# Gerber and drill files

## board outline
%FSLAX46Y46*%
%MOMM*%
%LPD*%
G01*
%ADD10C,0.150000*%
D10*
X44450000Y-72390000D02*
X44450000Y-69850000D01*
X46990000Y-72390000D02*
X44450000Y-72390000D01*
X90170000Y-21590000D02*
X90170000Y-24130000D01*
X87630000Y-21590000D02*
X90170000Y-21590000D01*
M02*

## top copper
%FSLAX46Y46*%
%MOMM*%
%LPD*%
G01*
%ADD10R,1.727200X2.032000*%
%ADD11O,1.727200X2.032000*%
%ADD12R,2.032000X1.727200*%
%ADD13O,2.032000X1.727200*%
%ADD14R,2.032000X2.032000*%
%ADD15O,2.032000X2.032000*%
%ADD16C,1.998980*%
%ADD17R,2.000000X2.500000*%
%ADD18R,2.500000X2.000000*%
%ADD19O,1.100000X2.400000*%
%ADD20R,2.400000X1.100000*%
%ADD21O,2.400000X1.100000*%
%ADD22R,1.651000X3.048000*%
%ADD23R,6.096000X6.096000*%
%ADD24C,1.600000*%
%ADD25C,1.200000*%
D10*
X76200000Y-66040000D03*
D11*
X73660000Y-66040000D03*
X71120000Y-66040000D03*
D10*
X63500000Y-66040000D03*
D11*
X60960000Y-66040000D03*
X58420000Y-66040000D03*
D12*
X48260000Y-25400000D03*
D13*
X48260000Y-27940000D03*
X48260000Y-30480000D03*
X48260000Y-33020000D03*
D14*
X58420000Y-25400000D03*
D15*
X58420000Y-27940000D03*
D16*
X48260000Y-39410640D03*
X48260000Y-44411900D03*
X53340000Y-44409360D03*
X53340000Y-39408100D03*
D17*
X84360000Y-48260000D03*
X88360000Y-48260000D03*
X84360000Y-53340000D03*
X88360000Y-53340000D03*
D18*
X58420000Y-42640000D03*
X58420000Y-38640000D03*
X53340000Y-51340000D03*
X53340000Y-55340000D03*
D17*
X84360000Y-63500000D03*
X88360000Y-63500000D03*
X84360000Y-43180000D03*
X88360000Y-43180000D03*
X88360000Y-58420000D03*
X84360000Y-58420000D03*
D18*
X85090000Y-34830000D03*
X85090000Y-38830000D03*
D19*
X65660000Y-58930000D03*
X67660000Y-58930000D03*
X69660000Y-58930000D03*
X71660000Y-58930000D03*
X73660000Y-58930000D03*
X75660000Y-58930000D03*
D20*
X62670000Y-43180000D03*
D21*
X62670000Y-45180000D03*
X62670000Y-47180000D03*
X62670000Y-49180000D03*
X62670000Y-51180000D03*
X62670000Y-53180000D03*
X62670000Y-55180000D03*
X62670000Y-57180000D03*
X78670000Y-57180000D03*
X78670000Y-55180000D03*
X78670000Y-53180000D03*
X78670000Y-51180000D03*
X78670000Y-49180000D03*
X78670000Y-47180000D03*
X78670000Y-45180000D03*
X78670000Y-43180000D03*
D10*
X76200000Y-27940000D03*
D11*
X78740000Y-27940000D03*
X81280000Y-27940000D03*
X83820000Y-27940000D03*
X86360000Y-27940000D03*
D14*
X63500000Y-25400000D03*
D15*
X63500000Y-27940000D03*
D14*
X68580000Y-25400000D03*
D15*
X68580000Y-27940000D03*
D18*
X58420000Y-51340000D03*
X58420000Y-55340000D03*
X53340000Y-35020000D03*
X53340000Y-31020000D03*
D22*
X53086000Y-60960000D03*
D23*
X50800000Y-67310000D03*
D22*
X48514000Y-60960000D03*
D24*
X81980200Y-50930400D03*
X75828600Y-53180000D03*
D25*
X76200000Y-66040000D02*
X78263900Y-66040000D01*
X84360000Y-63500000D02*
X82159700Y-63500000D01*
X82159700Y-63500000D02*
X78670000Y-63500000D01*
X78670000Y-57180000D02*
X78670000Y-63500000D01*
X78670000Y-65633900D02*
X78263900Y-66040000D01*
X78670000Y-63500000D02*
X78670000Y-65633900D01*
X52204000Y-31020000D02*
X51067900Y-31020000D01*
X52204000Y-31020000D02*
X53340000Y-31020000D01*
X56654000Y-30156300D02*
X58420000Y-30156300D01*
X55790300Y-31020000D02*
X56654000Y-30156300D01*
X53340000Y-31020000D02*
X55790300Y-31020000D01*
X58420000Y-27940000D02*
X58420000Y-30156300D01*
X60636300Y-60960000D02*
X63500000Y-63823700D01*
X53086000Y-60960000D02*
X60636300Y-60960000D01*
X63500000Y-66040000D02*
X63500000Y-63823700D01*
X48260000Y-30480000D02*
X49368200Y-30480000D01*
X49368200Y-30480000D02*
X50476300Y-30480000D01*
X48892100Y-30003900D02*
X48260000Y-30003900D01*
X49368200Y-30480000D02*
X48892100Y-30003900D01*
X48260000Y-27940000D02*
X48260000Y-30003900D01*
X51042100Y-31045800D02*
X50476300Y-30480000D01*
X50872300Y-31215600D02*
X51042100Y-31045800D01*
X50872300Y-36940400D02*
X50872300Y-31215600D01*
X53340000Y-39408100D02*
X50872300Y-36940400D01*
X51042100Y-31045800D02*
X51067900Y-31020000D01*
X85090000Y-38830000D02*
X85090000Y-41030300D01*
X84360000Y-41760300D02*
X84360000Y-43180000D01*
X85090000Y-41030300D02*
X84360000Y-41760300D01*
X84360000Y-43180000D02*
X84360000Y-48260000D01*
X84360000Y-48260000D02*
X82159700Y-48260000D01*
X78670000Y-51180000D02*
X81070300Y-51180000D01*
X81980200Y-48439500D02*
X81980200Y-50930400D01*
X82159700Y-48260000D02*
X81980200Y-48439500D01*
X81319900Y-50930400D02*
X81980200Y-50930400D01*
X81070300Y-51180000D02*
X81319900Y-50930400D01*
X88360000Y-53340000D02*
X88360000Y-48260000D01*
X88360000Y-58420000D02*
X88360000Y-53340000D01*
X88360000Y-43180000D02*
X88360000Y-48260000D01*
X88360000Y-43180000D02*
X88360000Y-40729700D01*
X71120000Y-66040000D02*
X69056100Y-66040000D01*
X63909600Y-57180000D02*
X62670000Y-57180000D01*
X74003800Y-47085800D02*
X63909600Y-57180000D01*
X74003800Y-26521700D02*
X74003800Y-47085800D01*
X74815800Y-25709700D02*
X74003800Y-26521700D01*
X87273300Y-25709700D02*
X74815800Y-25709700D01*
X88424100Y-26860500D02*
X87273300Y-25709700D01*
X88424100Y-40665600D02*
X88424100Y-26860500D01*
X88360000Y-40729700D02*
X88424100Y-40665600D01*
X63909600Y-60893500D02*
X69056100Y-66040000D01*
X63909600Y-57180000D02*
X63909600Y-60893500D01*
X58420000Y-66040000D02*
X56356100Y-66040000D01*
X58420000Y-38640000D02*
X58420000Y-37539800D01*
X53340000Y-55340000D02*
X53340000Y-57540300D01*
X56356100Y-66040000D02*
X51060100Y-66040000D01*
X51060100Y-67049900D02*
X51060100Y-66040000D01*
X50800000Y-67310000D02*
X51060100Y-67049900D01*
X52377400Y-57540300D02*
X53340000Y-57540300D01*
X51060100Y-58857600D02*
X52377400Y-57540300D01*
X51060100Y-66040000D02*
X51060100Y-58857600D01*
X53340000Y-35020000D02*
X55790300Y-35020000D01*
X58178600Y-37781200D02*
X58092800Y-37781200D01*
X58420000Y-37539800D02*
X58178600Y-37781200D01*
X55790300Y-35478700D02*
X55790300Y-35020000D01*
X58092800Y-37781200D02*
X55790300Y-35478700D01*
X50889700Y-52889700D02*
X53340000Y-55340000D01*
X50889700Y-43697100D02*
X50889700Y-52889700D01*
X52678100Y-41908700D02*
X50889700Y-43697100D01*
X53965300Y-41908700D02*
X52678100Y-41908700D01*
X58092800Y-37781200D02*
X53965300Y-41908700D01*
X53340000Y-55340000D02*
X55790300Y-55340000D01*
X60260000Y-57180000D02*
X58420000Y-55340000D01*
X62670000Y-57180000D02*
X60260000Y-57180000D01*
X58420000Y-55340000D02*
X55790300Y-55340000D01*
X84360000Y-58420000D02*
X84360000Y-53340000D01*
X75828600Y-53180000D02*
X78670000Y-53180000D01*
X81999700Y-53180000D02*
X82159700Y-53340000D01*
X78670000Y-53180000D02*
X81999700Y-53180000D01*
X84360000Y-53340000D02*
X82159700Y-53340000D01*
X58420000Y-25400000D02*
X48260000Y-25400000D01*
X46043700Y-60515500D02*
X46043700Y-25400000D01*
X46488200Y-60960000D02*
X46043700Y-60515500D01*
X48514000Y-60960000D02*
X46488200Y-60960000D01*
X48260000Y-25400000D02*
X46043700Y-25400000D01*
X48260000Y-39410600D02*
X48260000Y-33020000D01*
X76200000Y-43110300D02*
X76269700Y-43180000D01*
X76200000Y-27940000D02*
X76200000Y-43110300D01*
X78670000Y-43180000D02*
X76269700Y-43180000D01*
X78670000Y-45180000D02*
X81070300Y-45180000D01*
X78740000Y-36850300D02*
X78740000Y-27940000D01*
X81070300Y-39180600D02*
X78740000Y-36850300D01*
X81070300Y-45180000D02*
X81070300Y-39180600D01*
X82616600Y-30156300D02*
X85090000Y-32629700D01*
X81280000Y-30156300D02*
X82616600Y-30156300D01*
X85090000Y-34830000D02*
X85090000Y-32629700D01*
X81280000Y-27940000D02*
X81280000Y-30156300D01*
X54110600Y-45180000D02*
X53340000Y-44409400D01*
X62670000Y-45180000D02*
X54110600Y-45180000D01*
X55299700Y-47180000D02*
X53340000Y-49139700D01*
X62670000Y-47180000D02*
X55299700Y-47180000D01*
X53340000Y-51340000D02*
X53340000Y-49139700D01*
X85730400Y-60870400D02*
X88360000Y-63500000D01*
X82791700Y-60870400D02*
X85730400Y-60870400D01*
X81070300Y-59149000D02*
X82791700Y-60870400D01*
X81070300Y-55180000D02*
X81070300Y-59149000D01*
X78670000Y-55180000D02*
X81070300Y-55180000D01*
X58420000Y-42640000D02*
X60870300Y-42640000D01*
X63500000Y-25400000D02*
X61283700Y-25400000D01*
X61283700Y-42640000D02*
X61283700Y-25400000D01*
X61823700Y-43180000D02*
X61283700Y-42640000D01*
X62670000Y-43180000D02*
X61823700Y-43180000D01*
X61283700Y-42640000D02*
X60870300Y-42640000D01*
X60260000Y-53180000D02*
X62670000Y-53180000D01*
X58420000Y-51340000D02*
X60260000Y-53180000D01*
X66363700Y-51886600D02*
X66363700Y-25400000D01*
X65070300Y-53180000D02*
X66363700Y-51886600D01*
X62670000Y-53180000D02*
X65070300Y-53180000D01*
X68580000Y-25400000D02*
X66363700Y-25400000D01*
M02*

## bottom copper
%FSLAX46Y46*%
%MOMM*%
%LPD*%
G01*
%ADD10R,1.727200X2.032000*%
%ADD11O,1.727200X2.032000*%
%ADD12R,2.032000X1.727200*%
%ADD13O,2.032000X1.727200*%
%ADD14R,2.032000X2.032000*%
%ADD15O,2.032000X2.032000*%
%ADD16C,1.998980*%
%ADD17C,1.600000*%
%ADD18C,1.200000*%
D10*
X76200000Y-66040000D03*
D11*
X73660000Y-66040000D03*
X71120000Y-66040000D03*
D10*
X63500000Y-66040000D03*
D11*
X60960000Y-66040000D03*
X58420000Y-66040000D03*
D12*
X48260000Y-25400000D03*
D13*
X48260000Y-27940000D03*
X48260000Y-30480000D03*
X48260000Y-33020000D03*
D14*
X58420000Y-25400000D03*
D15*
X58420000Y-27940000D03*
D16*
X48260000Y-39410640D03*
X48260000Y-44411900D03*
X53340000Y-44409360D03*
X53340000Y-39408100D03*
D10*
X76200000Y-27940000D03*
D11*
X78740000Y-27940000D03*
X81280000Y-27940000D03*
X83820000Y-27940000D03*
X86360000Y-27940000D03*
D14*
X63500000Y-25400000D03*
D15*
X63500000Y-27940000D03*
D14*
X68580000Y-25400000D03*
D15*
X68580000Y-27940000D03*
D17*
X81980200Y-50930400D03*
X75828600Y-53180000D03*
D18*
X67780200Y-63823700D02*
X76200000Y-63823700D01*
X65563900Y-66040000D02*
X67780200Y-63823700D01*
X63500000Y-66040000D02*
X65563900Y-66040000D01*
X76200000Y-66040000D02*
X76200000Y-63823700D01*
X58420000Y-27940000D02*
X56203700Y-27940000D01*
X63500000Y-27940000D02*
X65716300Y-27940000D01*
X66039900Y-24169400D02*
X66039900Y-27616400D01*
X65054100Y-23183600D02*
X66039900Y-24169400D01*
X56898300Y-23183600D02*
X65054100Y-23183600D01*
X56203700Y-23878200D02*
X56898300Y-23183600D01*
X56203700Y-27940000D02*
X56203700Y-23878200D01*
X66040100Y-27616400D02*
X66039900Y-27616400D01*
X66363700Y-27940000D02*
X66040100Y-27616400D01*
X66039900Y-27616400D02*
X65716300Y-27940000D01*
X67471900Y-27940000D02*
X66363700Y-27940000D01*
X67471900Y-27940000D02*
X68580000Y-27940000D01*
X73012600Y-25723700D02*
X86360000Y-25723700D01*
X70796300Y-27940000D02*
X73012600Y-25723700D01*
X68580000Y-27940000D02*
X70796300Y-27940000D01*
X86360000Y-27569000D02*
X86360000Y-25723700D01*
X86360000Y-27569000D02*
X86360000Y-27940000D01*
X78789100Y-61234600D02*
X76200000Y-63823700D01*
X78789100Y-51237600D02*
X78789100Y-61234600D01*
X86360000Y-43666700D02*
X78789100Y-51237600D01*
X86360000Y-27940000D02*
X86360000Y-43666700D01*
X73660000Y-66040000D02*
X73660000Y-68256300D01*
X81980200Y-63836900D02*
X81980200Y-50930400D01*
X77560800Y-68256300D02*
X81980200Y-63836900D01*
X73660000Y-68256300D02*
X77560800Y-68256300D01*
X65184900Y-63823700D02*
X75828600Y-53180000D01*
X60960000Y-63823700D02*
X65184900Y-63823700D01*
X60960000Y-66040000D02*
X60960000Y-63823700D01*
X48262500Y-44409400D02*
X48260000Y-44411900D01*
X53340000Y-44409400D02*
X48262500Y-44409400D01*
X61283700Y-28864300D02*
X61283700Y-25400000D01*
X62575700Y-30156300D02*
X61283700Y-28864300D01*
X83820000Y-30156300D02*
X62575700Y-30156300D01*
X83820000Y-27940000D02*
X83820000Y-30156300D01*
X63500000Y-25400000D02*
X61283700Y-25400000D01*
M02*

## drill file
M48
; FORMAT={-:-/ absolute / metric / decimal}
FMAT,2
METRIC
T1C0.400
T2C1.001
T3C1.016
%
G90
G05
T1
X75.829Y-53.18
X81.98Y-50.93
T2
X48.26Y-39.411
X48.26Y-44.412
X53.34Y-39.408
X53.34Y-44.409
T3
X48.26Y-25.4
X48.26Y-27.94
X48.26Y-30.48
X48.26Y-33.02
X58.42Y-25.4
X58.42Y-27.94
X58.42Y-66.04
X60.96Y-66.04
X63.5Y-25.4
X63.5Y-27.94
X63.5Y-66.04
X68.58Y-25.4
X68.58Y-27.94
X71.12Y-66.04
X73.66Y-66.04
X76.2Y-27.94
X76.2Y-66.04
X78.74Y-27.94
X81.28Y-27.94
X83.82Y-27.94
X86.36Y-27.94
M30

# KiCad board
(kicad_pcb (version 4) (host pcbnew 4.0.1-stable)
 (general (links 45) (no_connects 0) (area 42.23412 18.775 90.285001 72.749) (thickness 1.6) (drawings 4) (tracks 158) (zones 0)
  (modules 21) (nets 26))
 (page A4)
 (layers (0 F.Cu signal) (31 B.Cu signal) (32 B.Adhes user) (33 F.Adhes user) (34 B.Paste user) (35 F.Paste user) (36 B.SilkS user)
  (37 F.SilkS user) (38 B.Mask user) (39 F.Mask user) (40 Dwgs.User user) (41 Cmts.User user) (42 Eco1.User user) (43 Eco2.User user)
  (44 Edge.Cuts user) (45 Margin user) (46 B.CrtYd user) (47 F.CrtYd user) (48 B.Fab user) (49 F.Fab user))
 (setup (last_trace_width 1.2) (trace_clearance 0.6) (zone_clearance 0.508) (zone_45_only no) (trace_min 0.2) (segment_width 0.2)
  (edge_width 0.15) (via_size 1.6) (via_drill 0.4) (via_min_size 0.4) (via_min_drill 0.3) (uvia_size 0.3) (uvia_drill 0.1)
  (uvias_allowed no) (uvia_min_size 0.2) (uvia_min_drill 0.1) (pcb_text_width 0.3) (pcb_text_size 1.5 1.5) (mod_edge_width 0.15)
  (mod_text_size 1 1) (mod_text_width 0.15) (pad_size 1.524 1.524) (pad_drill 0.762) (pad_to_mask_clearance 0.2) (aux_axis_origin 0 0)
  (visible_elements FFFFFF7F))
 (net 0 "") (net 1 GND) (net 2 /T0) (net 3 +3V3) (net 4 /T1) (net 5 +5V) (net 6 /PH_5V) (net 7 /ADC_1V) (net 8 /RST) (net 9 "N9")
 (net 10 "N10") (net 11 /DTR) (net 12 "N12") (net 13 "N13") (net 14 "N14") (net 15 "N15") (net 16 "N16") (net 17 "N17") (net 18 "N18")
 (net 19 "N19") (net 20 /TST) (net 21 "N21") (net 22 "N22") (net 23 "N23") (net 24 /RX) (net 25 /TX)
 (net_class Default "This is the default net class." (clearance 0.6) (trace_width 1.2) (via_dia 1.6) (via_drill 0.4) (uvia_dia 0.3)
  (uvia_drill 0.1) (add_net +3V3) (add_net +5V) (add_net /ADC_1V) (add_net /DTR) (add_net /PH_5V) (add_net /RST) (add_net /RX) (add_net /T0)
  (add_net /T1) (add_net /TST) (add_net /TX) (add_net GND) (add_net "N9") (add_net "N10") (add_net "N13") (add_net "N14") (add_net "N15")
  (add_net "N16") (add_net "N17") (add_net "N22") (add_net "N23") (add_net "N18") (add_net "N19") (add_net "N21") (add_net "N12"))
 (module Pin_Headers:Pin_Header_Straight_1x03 (layer F.Cu) (at 76.2 66.04 270)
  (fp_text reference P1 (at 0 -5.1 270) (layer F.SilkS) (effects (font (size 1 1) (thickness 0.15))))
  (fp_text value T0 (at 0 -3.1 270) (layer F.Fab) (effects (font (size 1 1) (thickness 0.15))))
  (pad 1 thru_hole rect (at 0 0 270) (size 2.032 1.7272) (drill 1.016) (layers *.Cu *.Mask F.SilkS) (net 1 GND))
  (pad 2 thru_hole oval (at 0 2.54 270) (size 2.032 1.7272) (drill 1.016) (layers *.Cu *.Mask F.SilkS) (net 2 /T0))
  (pad 3 thru_hole oval (at 0 5.08 270) (size 2.032 1.7272) (drill 1.016) (layers *.Cu *.Mask F.SilkS) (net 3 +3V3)))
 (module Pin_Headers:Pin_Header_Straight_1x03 (layer F.Cu) (at 63.5 66.04 270)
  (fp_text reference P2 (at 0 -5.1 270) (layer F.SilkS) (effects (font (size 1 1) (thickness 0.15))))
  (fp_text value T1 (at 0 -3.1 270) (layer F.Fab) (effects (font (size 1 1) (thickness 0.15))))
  (pad 1 thru_hole rect (at 0 0 270) (size 2.032 1.7272) (drill 1.016) (layers *.Cu *.Mask F.SilkS) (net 1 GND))
  (pad 2 thru_hole oval (at 0 2.54 270) (size 2.032 1.7272) (drill 1.016) (layers *.Cu *.Mask F.SilkS) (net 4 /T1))
  (pad 3 thru_hole oval (at 0 5.08 270) (size 2.032 1.7272) (drill 1.016) (layers *.Cu *.Mask F.SilkS) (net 3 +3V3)))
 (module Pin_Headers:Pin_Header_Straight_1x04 (layer F.Cu) (at 48.26 25.4)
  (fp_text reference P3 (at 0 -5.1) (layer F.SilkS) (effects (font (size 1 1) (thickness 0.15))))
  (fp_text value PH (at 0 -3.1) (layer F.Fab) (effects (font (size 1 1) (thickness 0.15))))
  (pad 1 thru_hole rect (at 0 0) (size 2.032 1.7272) (drill 1.016) (layers *.Cu *.Mask F.SilkS) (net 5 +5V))
  (pad 2 thru_hole oval (at 0 2.54) (size 2.032 1.7272) (drill 1.016) (layers *.Cu *.Mask F.SilkS) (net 1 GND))
  (pad 3 thru_hole oval (at 0 5.08) (size 2.032 1.7272) (drill 1.016) (layers *.Cu *.Mask F.SilkS) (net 1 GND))
  (pad 4 thru_hole oval (at 0 7.62) (size 2.032 1.7272) (drill 1.016) (layers *.Cu *.Mask F.SilkS) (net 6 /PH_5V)))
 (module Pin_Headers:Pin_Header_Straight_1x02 (layer F.Cu) (at 58.42 25.4)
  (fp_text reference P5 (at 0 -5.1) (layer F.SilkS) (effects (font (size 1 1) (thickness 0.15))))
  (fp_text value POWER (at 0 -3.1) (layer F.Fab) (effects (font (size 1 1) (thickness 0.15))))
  (pad 1 thru_hole rect (at 0 0) (size 2.032 2.032) (drill 1.016) (layers *.Cu *.Mask F.SilkS) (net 5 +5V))
  (pad 2 thru_hole oval (at 0 2.54) (size 2.032 2.032) (drill 1.016) (layers *.Cu *.Mask F.SilkS) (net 1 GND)))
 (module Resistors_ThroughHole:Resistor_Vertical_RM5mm (layer F.Cu) (at 48.26 41.91 270)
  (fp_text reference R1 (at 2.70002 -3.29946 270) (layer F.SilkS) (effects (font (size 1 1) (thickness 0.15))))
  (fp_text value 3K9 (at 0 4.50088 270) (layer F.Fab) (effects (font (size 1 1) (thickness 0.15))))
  (pad 1 thru_hole circle (at -2.49936 0 270) (size 1.99898 1.99898) (drill 1.00076) (layers *.Cu *.SilkS *.Mask) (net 6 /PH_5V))
  (pad 2 thru_hole circle (at 2.5019 0 270) (size 1.99898 1.99898) (drill 1.00076) (layers *.Cu *.SilkS *.Mask) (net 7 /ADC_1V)))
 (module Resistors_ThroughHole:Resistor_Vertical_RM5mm (layer F.Cu) (at 53.34 41.91 90)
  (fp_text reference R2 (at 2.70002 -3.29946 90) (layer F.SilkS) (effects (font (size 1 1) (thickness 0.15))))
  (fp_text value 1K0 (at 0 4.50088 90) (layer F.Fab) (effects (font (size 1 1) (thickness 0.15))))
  (pad 1 thru_hole circle (at -2.49936 0 90) (size 1.99898 1.99898) (drill 1.00076) (layers *.Cu *.SilkS *.Mask) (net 7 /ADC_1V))
  (pad 2 thru_hole circle (at 2.5019 0 90) (size 1.99898 1.99898) (drill 1.00076) (layers *.Cu *.SilkS *.Mask) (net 1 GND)))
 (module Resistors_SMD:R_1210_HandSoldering (layer F.Cu) (at 86.36 48.26)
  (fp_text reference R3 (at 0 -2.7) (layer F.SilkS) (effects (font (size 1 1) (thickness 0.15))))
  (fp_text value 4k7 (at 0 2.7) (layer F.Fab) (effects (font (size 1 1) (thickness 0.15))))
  (pad 1 smd rect (at -2 0) (size 2 2.5) (layers F.Cu F.Paste F.Mask) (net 2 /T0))
  (pad 2 smd rect (at 2 0) (size 2 2.5) (layers F.Cu F.Paste F.Mask) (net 3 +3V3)))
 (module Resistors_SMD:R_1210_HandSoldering (layer F.Cu) (at 86.36 53.34)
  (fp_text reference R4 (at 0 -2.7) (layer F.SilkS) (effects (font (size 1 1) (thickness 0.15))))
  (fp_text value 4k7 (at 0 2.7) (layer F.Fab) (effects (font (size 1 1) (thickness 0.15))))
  (pad 1 smd rect (at -2 0) (size 2 2.5) (layers F.Cu F.Paste F.Mask) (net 4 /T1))
  (pad 2 smd rect (at 2 0) (size 2 2.5) (layers F.Cu F.Paste F.Mask) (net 3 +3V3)))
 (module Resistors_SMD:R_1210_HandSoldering (layer F.Cu) (at 58.42 40.64 90)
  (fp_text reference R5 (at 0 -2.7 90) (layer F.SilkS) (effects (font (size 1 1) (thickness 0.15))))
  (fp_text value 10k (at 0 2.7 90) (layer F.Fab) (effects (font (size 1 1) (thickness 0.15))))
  (pad 1 smd rect (at -2 0 90) (size 2 2.5) (layers F.Cu F.Paste F.Mask) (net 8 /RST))
  (pad 2 smd rect (at 2 0 90) (size 2 2.5) (layers F.Cu F.Paste F.Mask) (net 3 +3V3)))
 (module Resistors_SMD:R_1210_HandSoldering (layer F.Cu) (at 53.34 53.34 270)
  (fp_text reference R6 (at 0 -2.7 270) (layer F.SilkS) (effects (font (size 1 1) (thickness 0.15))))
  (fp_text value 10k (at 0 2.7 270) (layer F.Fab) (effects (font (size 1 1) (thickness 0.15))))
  (pad 1 smd rect (at -2 0 270) (size 2 2.5) (layers F.Cu F.Paste F.Mask) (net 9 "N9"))
  (pad 2 smd rect (at 2 0 270) (size 2 2.5) (layers F.Cu F.Paste F.Mask) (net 3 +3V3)))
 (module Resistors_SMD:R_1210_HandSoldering (layer F.Cu) (at 86.36 63.5)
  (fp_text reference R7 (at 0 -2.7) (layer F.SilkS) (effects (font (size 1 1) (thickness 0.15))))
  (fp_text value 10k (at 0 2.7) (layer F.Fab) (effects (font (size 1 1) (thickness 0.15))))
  (pad 1 smd rect (at -2 0) (size 2 2.5) (layers F.Cu F.Paste F.Mask) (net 1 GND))
  (pad 2 smd rect (at 2 0) (size 2 2.5) (layers F.Cu F.Paste F.Mask) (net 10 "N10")))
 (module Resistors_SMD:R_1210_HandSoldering (layer F.Cu) (at 86.36 43.18)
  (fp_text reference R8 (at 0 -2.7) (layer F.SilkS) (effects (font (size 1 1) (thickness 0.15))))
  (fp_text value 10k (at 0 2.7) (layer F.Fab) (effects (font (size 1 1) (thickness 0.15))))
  (pad 1 smd rect (at -2 0) (size 2 2.5) (layers F.Cu F.Paste F.Mask) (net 2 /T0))
  (pad 2 smd rect (at 2 0) (size 2 2.5) (layers F.Cu F.Paste F.Mask) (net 3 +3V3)))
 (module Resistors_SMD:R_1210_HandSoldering (layer F.Cu) (at 86.36 58.42 180)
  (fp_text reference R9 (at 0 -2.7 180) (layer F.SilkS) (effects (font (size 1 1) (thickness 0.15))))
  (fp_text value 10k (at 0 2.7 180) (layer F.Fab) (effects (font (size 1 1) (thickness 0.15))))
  (pad 1 smd rect (at -2 0 180) (size 2 2.5) (layers F.Cu F.Paste F.Mask) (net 3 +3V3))
  (pad 2 smd rect (at 2 0 180) (size 2 2.5) (layers F.Cu F.Paste F.Mask) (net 4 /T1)))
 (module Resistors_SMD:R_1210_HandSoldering (layer F.Cu) (at 85.09 36.83 270)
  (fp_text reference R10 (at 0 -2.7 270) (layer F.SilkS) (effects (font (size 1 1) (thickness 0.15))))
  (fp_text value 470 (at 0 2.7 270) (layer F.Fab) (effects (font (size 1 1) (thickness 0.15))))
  (pad 1 smd rect (at -2 0 270) (size 2 2.5) (layers F.Cu F.Paste F.Mask) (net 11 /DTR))
  (pad 2 smd rect (at 2 0 270) (size 2 2.5) (layers F.Cu F.Paste F.Mask) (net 2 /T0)))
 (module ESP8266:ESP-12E (layer F.Cu) (at 62.67 43.18)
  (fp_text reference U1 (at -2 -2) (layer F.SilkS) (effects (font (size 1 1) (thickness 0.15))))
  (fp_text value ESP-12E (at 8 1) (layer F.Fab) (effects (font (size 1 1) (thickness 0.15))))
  (pad 9 smd oval (at 2.99 15.75 90) (size 2.4 1.1) (layers F.Cu F.Paste F.Mask) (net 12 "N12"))
  (pad 10 smd oval (at 4.99 15.75 90) (size 2.4 1.1) (layers F.Cu F.Paste F.Mask) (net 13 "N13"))
  (pad 11 smd oval (at 6.99 15.75 90) (size 2.4 1.1) (layers F.Cu F.Paste F.Mask) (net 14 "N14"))
  (pad 12 smd oval (at 8.99 15.75 90) (size 2.4 1.1) (layers F.Cu F.Paste F.Mask) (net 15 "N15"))
  (pad 13 smd oval (at 10.99 15.75 90) (size 2.4 1.1) (layers F.Cu F.Paste F.Mask) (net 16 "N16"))
  (pad 14 smd oval (at 12.99 15.75 90) (size 2.4 1.1) (layers F.Cu F.Paste F.Mask) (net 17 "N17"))
  (pad 1 smd rect (at 0 0) (size 2.4 1.1) (layers F.Cu F.Paste F.Mask) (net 8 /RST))
  (pad 2 smd oval (at 0 2) (size 2.4 1.1) (layers F.Cu F.Paste F.Mask) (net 7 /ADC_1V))
  (pad 3 smd oval (at 0 4) (size 2.4 1.1) (layers F.Cu F.Paste F.Mask) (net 9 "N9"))
  (pad 4 smd oval (at 0 6) (size 2.4 1.1) (layers F.Cu F.Paste F.Mask) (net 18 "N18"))
  (pad 5 smd oval (at 0 8) (size 2.4 1.1) (layers F.Cu F.Paste F.Mask) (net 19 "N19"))
  (pad 6 smd oval (at 0 10) (size 2.4 1.1) (layers F.Cu F.Paste F.Mask) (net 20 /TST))
  (pad 7 smd oval (at 0 12) (size 2.4 1.1) (layers F.Cu F.Paste F.Mask) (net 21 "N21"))
  (pad 8 smd oval (at 0 14) (size 2.4 1.1) (layers F.Cu F.Paste F.Mask) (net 3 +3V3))
  (pad 15 smd oval (at 16 14) (size 2.4 1.1) (layers F.Cu F.Paste F.Mask) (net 1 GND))
  (pad 16 smd oval (at 16 12) (size 2.4 1.1) (layers F.Cu F.Paste F.Mask) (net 10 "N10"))
  (pad 17 smd oval (at 16 10) (size 2.4 1.1) (layers F.Cu F.Paste F.Mask) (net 4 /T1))
  (pad 18 smd oval (at 16 8) (size 2.4 1.1) (layers F.Cu F.Paste F.Mask) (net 2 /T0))
  (pad 19 smd oval (at 16 6) (size 2.4 1.1) (layers F.Cu F.Paste F.Mask) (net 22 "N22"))
  (pad 20 smd oval (at 16 4) (size 2.4 1.1) (layers F.Cu F.Paste F.Mask) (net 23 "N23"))
  (pad 21 smd oval (at 16 2) (size 2.4 1.1) (layers F.Cu F.Paste F.Mask) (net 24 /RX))
  (pad 22 smd oval (at 16 0) (size 2.4 1.1) (layers F.Cu F.Paste F.Mask) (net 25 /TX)))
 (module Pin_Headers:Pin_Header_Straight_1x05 (layer F.Cu) (at 76.2 27.94 90)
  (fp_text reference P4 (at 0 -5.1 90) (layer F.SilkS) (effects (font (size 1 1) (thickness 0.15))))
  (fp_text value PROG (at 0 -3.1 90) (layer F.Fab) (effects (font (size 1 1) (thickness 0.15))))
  (pad 1 thru_hole rect (at 0 0 90) (size 2.032 1.7272) (drill 1.016) (layers *.Cu *.Mask F.SilkS) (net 25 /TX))
  (pad 2 thru_hole oval (at 0 2.54 90) (size 2.032 1.7272) (drill 1.016) (layers *.Cu *.Mask F.SilkS) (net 24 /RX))
  (pad 3 thru_hole oval (at 0 5.08 90) (size 2.032 1.7272) (drill 1.016) (layers *.Cu *.Mask F.SilkS) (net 11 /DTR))
  (pad 4 thru_hole oval (at 0 7.62 90) (size 2.032 1.7272) (drill 1.016) (layers *.Cu *.Mask F.SilkS) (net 8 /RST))
  (pad 5 thru_hole oval (at 0 10.16 90) (size 2.032 1.7272) (drill 1.016) (layers *.Cu *.Mask F.SilkS) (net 1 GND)))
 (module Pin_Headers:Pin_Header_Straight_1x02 (layer F.Cu) (at 63.5 25.4)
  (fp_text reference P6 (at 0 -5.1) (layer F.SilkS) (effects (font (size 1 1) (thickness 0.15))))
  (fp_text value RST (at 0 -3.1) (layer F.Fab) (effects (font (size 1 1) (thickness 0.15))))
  (pad 1 thru_hole rect (at 0 0) (size 2.032 2.032) (drill 1.016) (layers *.Cu *.Mask F.SilkS) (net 8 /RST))
  (pad 2 thru_hole oval (at 0 2.54) (size 2.032 2.032) (drill 1.016) (layers *.Cu *.Mask F.SilkS) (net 1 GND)))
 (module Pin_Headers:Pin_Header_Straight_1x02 (layer F.Cu) (at 68.58 25.4)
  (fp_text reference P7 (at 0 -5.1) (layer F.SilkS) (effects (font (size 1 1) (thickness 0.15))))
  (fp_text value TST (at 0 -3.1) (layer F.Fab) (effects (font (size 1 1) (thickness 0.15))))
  (pad 1 thru_hole rect (at 0 0) (size 2.032 2.032) (drill 1.016) (layers *.Cu *.Mask F.SilkS) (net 20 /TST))
  (pad 2 thru_hole oval (at 0 2.54) (size 2.032 2.032) (drill 1.016) (layers *.Cu *.Mask F.SilkS) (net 1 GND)))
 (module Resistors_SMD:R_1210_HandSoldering (layer F.Cu) (at 58.42 53.34 270)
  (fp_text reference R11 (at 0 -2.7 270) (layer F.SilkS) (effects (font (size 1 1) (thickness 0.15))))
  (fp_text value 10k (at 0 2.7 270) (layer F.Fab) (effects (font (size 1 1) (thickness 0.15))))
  (pad 1 smd rect (at -2 0 270) (size 2 2.5) (layers F.Cu F.Paste F.Mask) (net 20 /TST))
  (pad 2 smd rect (at 2 0 270) (size 2 2.5) (layers F.Cu F.Paste F.Mask) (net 3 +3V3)))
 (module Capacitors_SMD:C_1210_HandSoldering (layer F.Cu) (at 53.34 33.02 90)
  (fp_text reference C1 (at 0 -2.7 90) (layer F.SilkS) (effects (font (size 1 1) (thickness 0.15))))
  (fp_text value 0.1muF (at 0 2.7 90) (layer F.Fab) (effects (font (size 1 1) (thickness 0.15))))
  (pad 1 smd rect (at -2 0 90) (size 2 2.5) (layers F.Cu F.Paste F.Mask) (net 3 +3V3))
  (pad 2 smd rect (at 2 0 90) (size 2 2.5) (layers F.Cu F.Paste F.Mask) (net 1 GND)))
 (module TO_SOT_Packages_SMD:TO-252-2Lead (layer F.Cu) (at 50.8 60.96 180)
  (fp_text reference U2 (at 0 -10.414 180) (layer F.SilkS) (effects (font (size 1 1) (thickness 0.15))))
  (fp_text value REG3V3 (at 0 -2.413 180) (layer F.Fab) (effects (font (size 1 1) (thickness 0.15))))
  (pad 1 smd rect (at -2.286 0 180) (size 1.651 3.048) (layers F.Cu F.Paste F.Mask) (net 1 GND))
  (pad 2 smd rect (at 0 -6.35 180) (size 6.096 6.096) (layers F.Cu F.Paste F.Mask) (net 3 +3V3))
  (pad 3 smd rect (at 2.286 0 180) (size 1.651 3.048) (layers F.Cu F.Paste F.Mask) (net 5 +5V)))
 (gr_line (start 44.45 72.39) (end 44.45 69.85) (angle 90) (layer Edge.Cuts) (width 0.15))
 (gr_line (start 46.99 72.39) (end 44.45 72.39) (angle 90) (layer Edge.Cuts) (width 0.15))
 (gr_line (start 90.17 21.59) (end 90.17 24.13) (angle 90) (layer Edge.Cuts) (width 0.15))
 (gr_line (start 87.63 21.59) (end 90.17 21.59) (angle 90) (layer Edge.Cuts) (width 0.15))
 (segment (start 76.2 66.04) (end 78.2639 66.04) (width 1.2) (layer F.Cu) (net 1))
 (segment (start 84.36 63.5) (end 82.1597 63.5) (width 1.2) (layer F.Cu) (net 1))
 (segment (start 82.1597 63.5) (end 78.67 63.5) (width 1.2) (layer F.Cu) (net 1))
 (segment (start 78.67 57.18) (end 78.67 63.5) (width 1.2) (layer F.Cu) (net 1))
 (segment (start 78.67 65.6339) (end 78.2639 66.04) (width 1.2) (layer F.Cu) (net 1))
 (segment (start 78.67 63.5) (end 78.67 65.6339) (width 1.2) (layer F.Cu) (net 1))
 (segment (start 67.7802 63.8237) (end 76.2 63.8237) (width 1.2) (layer B.Cu) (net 1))
 (segment (start 65.5639 66.04) (end 67.7802 63.8237) (width 1.2) (layer B.Cu) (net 1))
 (segment (start 63.5 66.04) (end 65.5639 66.04) (width 1.2) (layer B.Cu) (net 1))
 (segment (start 76.2 66.04) (end 76.2 63.8237) (width 1.2) (layer B.Cu) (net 1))
 (segment (start 58.42 27.94) (end 56.2037 27.94) (width 1.2) (layer B.Cu) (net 1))
 (segment (start 63.5 27.94) (end 65.7163 27.94) (width 1.2) (layer B.Cu) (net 1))
 (segment (start 66.0399 24.1694) (end 66.0399 27.6164) (width 1.2) (layer B.Cu) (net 1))
 (segment (start 65.0541 23.1836) (end 66.0399 24.1694) (width 1.2) (layer B.Cu) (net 1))
 (segment (start 56.8983 23.1836) (end 65.0541 23.1836) (width 1.2) (layer B.Cu) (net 1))
 (segment (start 56.2037 23.8782) (end 56.8983 23.1836) (width 1.2) (layer B.Cu) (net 1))
 (segment (start 56.2037 27.94) (end 56.2037 23.8782) (width 1.2) (layer B.Cu) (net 1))
 (segment (start 66.0401 27.6164) (end 66.0399 27.6164) (width 1.2) (layer B.Cu) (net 1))
 (segment (start 66.3637 27.94) (end 66.0401 27.6164) (width 1.2) (layer B.Cu) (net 1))
 (segment (start 66.0399 27.6164) (end 65.7163 27.94) (width 1.2) (layer B.Cu) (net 1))
 (segment (start 67.4719 27.94) (end 66.3637 27.94) (width 1.2) (layer B.Cu) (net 1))
 (segment (start 67.4719 27.94) (end 68.58 27.94) (width 1.2) (layer B.Cu) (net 1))
 (segment (start 73.0126 25.7237) (end 86.36 25.7237) (width 1.2) (layer B.Cu) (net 1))
 (segment (start 70.7963 27.94) (end 73.0126 25.7237) (width 1.2) (layer B.Cu) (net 1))
 (segment (start 68.58 27.94) (end 70.7963 27.94) (width 1.2) (layer B.Cu) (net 1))
 (segment (start 52.204 31.02) (end 51.0679 31.02) (width 1.2) (layer F.Cu) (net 1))
 (segment (start 52.204 31.02) (end 53.34 31.02) (width 1.2) (layer F.Cu) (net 1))
 (segment (start 56.654 30.1563) (end 58.42 30.1563) (width 1.2) (layer F.Cu) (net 1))
 (segment (start 55.7903 31.02) (end 56.654 30.1563) (width 1.2) (layer F.Cu) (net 1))
 (segment (start 53.34 31.02) (end 55.7903 31.02) (width 1.2) (layer F.Cu) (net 1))
 (segment (start 58.42 27.94) (end 58.42 30.1563) (width 1.2) (layer F.Cu) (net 1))
 (segment (start 60.6363 60.96) (end 63.5 63.8237) (width 1.2) (layer F.Cu) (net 1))
 (segment (start 53.086 60.96) (end 60.6363 60.96) (width 1.2) (layer F.Cu) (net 1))
 (segment (start 63.5 66.04) (end 63.5 63.8237) (width 1.2) (layer F.Cu) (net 1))
 (segment (start 86.36 27.569) (end 86.36 25.7237) (width 1.2) (layer B.Cu) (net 1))
 (segment (start 86.36 27.569) (end 86.36 27.94) (width 1.2) (layer B.Cu) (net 1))
 (segment (start 78.7891 61.2346) (end 76.2 63.8237) (width 1.2) (layer B.Cu) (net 1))
 (segment (start 78.7891 51.2376) (end 78.7891 61.2346) (width 1.2) (layer B.Cu) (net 1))
 (segment (start 86.36 43.6667) (end 78.7891 51.2376) (width 1.2) (layer B.Cu) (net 1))
 (segment (start 86.36 27.94) (end 86.36 43.6667) (width 1.2) (layer B.Cu) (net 1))
 (segment (start 48.26 30.48) (end 49.3682 30.48) (width 1.2) (layer F.Cu) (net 1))
 (segment (start 49.3682 30.48) (end 50.4763 30.48) (width 1.2) (layer F.Cu) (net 1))
 (segment (start 48.8921 30.0039) (end 48.26 30.0039) (width 1.2) (layer F.Cu) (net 1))
 (segment (start 49.3682 30.48) (end 48.8921 30.0039) (width 1.2) (layer F.Cu) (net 1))
 (segment (start 48.26 27.94) (end 48.26 30.0039) (width 1.2) (layer F.Cu) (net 1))
 (segment (start 51.0421 31.0458) (end 50.4763 30.48) (width 1.2) (layer F.Cu) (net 1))
 (segment (start 50.8723 31.2156) (end 51.0421 31.0458) (width 1.2) (layer F.Cu) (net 1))
 (segment (start 50.8723 36.9404) (end 50.8723 31.2156) (width 1.2) (layer F.Cu) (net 1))
 (segment (start 53.34 39.4081) (end 50.8723 36.9404) (width 1.2) (layer F.Cu) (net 1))
 (segment (start 51.0421 31.0458) (end 51.0679 31.02) (width 1.2) (layer F.Cu) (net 1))
 (via (at 81.9802 50.9304) (size 1.6) (layers F.Cu B.Cu) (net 2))
 (segment (start 85.09 38.83) (end 85.09 41.0303) (width 1.2) (layer F.Cu) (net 2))
 (segment (start 84.36 41.7603) (end 84.36 43.18) (width 1.2) (layer F.Cu) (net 2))
 (segment (start 85.09 41.0303) (end 84.36 41.7603) (width 1.2) (layer F.Cu) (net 2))
 (segment (start 84.36 43.18) (end 84.36 48.26) (width 1.2) (layer F.Cu) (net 2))
 (segment (start 84.36 48.26) (end 82.1597 48.26) (width 1.2) (layer F.Cu) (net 2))
 (segment (start 78.67 51.18) (end 81.0703 51.18) (width 1.2) (layer F.Cu) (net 2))
 (segment (start 73.66 66.04) (end 73.66 68.2563) (width 1.2) (layer B.Cu) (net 2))
 (segment (start 81.9802 48.4395) (end 81.9802 50.9304) (width 1.2) (layer F.Cu) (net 2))
 (segment (start 82.1597 48.26) (end 81.9802 48.4395) (width 1.2) (layer F.Cu) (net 2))
 (segment (start 81.3199 50.9304) (end 81.9802 50.9304) (width 1.2) (layer F.Cu) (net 2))
 (segment (start 81.0703 51.18) (end 81.3199 50.9304) (width 1.2) (layer F.Cu) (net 2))
 (segment (start 81.9802 63.8369) (end 81.9802 50.9304) (width 1.2) (layer B.Cu) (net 2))
 (segment (start 77.5608 68.2563) (end 81.9802 63.8369) (width 1.2) (layer B.Cu) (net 2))
 (segment (start 73.66 68.2563) (end 77.5608 68.2563) (width 1.2) (layer B.Cu) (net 2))
 (segment (start 88.36 53.34) (end 88.36 48.26) (width 1.2) (layer F.Cu) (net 3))
 (segment (start 88.36 58.42) (end 88.36 53.34) (width 1.2) (layer F.Cu) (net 3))
 (segment (start 88.36 43.18) (end 88.36 48.26) (width 1.2) (layer F.Cu) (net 3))
 (segment (start 88.36 43.18) (end 88.36 40.7297) (width 1.2) (layer F.Cu) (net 3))
 (segment (start 71.12 66.04) (end 69.0561 66.04) (width 1.2) (layer F.Cu) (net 3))
 (segment (start 63.9096 57.18) (end 62.67 57.18) (width 1.2) (layer F.Cu) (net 3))
 (segment (start 74.0038 47.0858) (end 63.9096 57.18) (width 1.2) (layer F.Cu) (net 3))
 (segment (start 74.0038 26.5217) (end 74.0038 47.0858) (width 1.2) (layer F.Cu) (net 3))
 (segment (start 74.8158 25.7097) (end 74.0038 26.5217) (width 1.2) (layer F.Cu) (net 3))
 (segment (start 87.2733 25.7097) (end 74.8158 25.7097) (width 1.2) (layer F.Cu) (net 3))
 (segment (start 88.4241 26.8605) (end 87.2733 25.7097) (width 1.2) (layer F.Cu) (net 3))
 (segment (start 88.4241 40.6656) (end 88.4241 26.8605) (width 1.2) (layer F.Cu) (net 3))
 (segment (start 88.36 40.7297) (end 88.4241 40.6656) (width 1.2) (layer F.Cu) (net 3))
 (segment (start 63.9096 60.8935) (end 69.0561 66.04) (width 1.2) (layer F.Cu) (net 3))
 (segment (start 63.9096 57.18) (end 63.9096 60.8935) (width 1.2) (layer F.Cu) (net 3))
 (segment (start 58.42 66.04) (end 56.3561 66.04) (width 1.2) (layer F.Cu) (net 3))
 (segment (start 58.42 38.64) (end 58.42 37.5398) (width 1.2) (layer F.Cu) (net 3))
 (segment (start 53.34 55.34) (end 53.34 57.5403) (width 1.2) (layer F.Cu) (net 3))
 (segment (start 56.3561 66.04) (end 51.0601 66.04) (width 1.2) (layer F.Cu) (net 3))
 (segment (start 51.0601 67.0499) (end 51.0601 66.04) (width 1.2) (layer F.Cu) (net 3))
 (segment (start 50.8 67.31) (end 51.0601 67.0499) (width 1.2) (layer F.Cu) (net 3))
 (segment (start 52.3774 57.5403) (end 53.34 57.5403) (width 1.2) (layer F.Cu) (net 3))
 (segment (start 51.0601 58.8576) (end 52.3774 57.5403) (width 1.2) (layer F.Cu) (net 3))
 (segment (start 51.0601 66.04) (end 51.0601 58.8576) (width 1.2) (layer F.Cu) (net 3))
 (segment (start 53.34 35.02) (end 55.7903 35.02) (width 1.2) (layer F.Cu) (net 3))
 (segment (start 58.1786 37.7812) (end 58.0928 37.7812) (width 1.2) (layer F.Cu) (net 3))
 (segment (start 58.42 37.5398) (end 58.1786 37.7812) (width 1.2) (layer F.Cu) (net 3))
 (segment (start 55.7903 35.4787) (end 55.7903 35.02) (width 1.2) (layer F.Cu) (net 3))
 (segment (start 58.0928 37.7812) (end 55.7903 35.4787) (width 1.2) (layer F.Cu) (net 3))
 (segment (start 50.8897 52.8897) (end 53.34 55.34) (width 1.2) (layer F.Cu) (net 3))
 (segment (start 50.8897 43.6971) (end 50.8897 52.8897) (width 1.2) (layer F.Cu) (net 3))
 (segment (start 52.6781 41.9087) (end 50.8897 43.6971) (width 1.2) (layer F.Cu) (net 3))
 (segment (start 53.9653 41.9087) (end 52.6781 41.9087) (width 1.2) (layer F.Cu) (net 3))
 (segment (start 58.0928 37.7812) (end 53.9653 41.9087) (width 1.2) (layer F.Cu) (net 3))
 (segment (start 53.34 55.34) (end 55.7903 55.34) (width 1.2) (layer F.Cu) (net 3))
 (segment (start 60.26 57.18) (end 58.42 55.34) (width 1.2) (layer F.Cu) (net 3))
 (segment (start 62.67 57.18) (end 60.26 57.18) (width 1.2) (layer F.Cu) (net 3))
 (segment (start 58.42 55.34) (end 55.7903 55.34) (width 1.2) (layer F.Cu) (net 3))
 (via (at 75.8286 53.18) (size 1.6) (layers F.Cu B.Cu) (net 4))
 (segment (start 65.1849 63.8237) (end 75.8286 53.18) (width 1.2) (layer B.Cu) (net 4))
 (segment (start 60.96 63.8237) (end 65.1849 63.8237) (width 1.2) (layer B.Cu) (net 4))
 (segment (start 60.96 66.04) (end 60.96 63.8237) (width 1.2) (layer B.Cu) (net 4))
 (segment (start 84.36 58.42) (end 84.36 53.34) (width 1.2) (layer F.Cu) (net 4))
 (segment (start 75.8286 53.18) (end 78.67 53.18) (width 1.2) (layer F.Cu) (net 4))
 (segment (start 81.9997 53.18) (end 82.1597 53.34) (width 1.2) (layer F.Cu) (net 4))
 (segment (start 78.67 53.18) (end 81.9997 53.18) (width 1.2) (layer F.Cu) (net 4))
 (segment (start 84.36 53.34) (end 82.1597 53.34) (width 1.2) (layer F.Cu) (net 4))
 (segment (start 58.42 25.4) (end 48.26 25.4) (width 1.2) (layer F.Cu) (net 5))
 (segment (start 46.0437 60.5155) (end 46.0437 25.4) (width 1.2) (layer F.Cu) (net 5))
 (segment (start 46.4882 60.96) (end 46.0437 60.5155) (width 1.2) (layer F.Cu) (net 5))
 (segment (start 48.514 60.96) (end 46.4882 60.96) (width 1.2) (layer F.Cu) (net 5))
 (segment (start 48.26 25.4) (end 46.0437 25.4) (width 1.2) (layer F.Cu) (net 5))
 (segment (start 48.26 39.4106) (end 48.26 33.02) (width 1.2) (layer F.Cu) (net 6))
 (segment (start 76.2 43.1103) (end 76.2697 43.18) (width 1.2) (layer F.Cu) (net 25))
 (segment (start 76.2 27.94) (end 76.2 43.1103) (width 1.2) (layer F.Cu) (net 25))
 (segment (start 78.67 43.18) (end 76.2697 43.18) (width 1.2) (layer F.Cu) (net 25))
 (segment (start 78.67 45.18) (end 81.0703 45.18) (width 1.2) (layer F.Cu) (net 24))
 (segment (start 78.74 36.8503) (end 78.74 27.94) (width 1.2) (layer F.Cu) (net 24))
 (segment (start 81.0703 39.1806) (end 78.74 36.8503) (width 1.2) (layer F.Cu) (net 24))
 (segment (start 81.0703 45.18) (end 81.0703 39.1806) (width 1.2) (layer F.Cu) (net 24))
 (segment (start 82.6166 30.1563) (end 85.09 32.6297) (width 1.2) (layer F.Cu) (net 11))
 (segment (start 81.28 30.1563) (end 82.6166 30.1563) (width 1.2) (layer F.Cu) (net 11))
 (segment (start 85.09 34.83) (end 85.09 32.6297) (width 1.2) (layer F.Cu) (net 11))
 (segment (start 81.28 27.94) (end 81.28 30.1563) (width 1.2) (layer F.Cu) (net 11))
 (segment (start 54.1106 45.18) (end 53.34 44.4094) (width 1.2) (layer F.Cu) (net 7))
 (segment (start 62.67 45.18) (end 54.1106 45.18) (width 1.2) (layer F.Cu) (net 7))
 (segment (start 48.2625 44.4094) (end 48.26 44.4119) (width 1.2) (layer B.Cu) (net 7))
 (segment (start 53.34 44.4094) (end 48.2625 44.4094) (width 1.2) (layer B.Cu) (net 7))
 (segment (start 55.2997 47.18) (end 53.34 49.1397) (width 1.2) (layer F.Cu) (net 9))
 (segment (start 62.67 47.18) (end 55.2997 47.18) (width 1.2) (layer F.Cu) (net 9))
 (segment (start 53.34 51.34) (end 53.34 49.1397) (width 1.2) (layer F.Cu) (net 9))
 (segment (start 85.7304 60.8704) (end 88.36 63.5) (width 1.2) (layer F.Cu) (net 10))
 (segment (start 82.7917 60.8704) (end 85.7304 60.8704) (width 1.2) (layer F.Cu) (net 10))
 (segment (start 81.0703 59.149) (end 82.7917 60.8704) (width 1.2) (layer F.Cu) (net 10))
 (segment (start 81.0703 55.18) (end 81.0703 59.149) (width 1.2) (layer F.Cu) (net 10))
 (segment (start 78.67 55.18) (end 81.0703 55.18) (width 1.2) (layer F.Cu) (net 10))
 (segment (start 61.2837 28.8643) (end 61.2837 25.4) (width 1.2) (layer B.Cu) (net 8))
 (segment (start 62.5757 30.1563) (end 61.2837 28.8643) (width 1.2) (layer B.Cu) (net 8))
 (segment (start 83.82 30.1563) (end 62.5757 30.1563) (width 1.2) (layer B.Cu) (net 8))
 (segment (start 83.82 27.94) (end 83.82 30.1563) (width 1.2) (layer B.Cu) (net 8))
 (segment (start 63.5 25.4) (end 61.2837 25.4) (width 1.2) (layer B.Cu) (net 8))
 (segment (start 58.42 42.64) (end 60.8703 42.64) (width 1.2) (layer F.Cu) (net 8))
 (segment (start 63.5 25.4) (end 61.2837 25.4) (width 1.2) (layer F.Cu) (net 8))
 (segment (start 61.2837 42.64) (end 61.2837 25.4) (width 1.2) (layer F.Cu) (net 8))
 (segment (start 61.8237 43.18) (end 61.2837 42.64) (width 1.2) (layer F.Cu) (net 8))
 (segment (start 62.67 43.18) (end 61.8237 43.18) (width 1.2) (layer F.Cu) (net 8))
 (segment (start 61.2837 42.64) (end 60.8703 42.64) (width 1.2) (layer F.Cu) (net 8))
 (segment (start 60.26 53.18) (end 62.67 53.18) (width 1.2) (layer F.Cu) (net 20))
 (segment (start 58.42 51.34) (end 60.26 53.18) (width 1.2) (layer F.Cu) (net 20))
 (segment (start 66.3637 51.8866) (end 66.3637 25.4) (width 1.2) (layer F.Cu) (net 20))
 (segment (start 65.0703 53.18) (end 66.3637 51.8866) (width 1.2) (layer F.Cu) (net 20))
 (segment (start 62.67 53.18) (end 65.0703 53.18) (width 1.2) (layer F.Cu) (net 20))
 (segment (start 68.58 25.4) (end 66.3637 25.4) (width 1.2) (layer F.Cu) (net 20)))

